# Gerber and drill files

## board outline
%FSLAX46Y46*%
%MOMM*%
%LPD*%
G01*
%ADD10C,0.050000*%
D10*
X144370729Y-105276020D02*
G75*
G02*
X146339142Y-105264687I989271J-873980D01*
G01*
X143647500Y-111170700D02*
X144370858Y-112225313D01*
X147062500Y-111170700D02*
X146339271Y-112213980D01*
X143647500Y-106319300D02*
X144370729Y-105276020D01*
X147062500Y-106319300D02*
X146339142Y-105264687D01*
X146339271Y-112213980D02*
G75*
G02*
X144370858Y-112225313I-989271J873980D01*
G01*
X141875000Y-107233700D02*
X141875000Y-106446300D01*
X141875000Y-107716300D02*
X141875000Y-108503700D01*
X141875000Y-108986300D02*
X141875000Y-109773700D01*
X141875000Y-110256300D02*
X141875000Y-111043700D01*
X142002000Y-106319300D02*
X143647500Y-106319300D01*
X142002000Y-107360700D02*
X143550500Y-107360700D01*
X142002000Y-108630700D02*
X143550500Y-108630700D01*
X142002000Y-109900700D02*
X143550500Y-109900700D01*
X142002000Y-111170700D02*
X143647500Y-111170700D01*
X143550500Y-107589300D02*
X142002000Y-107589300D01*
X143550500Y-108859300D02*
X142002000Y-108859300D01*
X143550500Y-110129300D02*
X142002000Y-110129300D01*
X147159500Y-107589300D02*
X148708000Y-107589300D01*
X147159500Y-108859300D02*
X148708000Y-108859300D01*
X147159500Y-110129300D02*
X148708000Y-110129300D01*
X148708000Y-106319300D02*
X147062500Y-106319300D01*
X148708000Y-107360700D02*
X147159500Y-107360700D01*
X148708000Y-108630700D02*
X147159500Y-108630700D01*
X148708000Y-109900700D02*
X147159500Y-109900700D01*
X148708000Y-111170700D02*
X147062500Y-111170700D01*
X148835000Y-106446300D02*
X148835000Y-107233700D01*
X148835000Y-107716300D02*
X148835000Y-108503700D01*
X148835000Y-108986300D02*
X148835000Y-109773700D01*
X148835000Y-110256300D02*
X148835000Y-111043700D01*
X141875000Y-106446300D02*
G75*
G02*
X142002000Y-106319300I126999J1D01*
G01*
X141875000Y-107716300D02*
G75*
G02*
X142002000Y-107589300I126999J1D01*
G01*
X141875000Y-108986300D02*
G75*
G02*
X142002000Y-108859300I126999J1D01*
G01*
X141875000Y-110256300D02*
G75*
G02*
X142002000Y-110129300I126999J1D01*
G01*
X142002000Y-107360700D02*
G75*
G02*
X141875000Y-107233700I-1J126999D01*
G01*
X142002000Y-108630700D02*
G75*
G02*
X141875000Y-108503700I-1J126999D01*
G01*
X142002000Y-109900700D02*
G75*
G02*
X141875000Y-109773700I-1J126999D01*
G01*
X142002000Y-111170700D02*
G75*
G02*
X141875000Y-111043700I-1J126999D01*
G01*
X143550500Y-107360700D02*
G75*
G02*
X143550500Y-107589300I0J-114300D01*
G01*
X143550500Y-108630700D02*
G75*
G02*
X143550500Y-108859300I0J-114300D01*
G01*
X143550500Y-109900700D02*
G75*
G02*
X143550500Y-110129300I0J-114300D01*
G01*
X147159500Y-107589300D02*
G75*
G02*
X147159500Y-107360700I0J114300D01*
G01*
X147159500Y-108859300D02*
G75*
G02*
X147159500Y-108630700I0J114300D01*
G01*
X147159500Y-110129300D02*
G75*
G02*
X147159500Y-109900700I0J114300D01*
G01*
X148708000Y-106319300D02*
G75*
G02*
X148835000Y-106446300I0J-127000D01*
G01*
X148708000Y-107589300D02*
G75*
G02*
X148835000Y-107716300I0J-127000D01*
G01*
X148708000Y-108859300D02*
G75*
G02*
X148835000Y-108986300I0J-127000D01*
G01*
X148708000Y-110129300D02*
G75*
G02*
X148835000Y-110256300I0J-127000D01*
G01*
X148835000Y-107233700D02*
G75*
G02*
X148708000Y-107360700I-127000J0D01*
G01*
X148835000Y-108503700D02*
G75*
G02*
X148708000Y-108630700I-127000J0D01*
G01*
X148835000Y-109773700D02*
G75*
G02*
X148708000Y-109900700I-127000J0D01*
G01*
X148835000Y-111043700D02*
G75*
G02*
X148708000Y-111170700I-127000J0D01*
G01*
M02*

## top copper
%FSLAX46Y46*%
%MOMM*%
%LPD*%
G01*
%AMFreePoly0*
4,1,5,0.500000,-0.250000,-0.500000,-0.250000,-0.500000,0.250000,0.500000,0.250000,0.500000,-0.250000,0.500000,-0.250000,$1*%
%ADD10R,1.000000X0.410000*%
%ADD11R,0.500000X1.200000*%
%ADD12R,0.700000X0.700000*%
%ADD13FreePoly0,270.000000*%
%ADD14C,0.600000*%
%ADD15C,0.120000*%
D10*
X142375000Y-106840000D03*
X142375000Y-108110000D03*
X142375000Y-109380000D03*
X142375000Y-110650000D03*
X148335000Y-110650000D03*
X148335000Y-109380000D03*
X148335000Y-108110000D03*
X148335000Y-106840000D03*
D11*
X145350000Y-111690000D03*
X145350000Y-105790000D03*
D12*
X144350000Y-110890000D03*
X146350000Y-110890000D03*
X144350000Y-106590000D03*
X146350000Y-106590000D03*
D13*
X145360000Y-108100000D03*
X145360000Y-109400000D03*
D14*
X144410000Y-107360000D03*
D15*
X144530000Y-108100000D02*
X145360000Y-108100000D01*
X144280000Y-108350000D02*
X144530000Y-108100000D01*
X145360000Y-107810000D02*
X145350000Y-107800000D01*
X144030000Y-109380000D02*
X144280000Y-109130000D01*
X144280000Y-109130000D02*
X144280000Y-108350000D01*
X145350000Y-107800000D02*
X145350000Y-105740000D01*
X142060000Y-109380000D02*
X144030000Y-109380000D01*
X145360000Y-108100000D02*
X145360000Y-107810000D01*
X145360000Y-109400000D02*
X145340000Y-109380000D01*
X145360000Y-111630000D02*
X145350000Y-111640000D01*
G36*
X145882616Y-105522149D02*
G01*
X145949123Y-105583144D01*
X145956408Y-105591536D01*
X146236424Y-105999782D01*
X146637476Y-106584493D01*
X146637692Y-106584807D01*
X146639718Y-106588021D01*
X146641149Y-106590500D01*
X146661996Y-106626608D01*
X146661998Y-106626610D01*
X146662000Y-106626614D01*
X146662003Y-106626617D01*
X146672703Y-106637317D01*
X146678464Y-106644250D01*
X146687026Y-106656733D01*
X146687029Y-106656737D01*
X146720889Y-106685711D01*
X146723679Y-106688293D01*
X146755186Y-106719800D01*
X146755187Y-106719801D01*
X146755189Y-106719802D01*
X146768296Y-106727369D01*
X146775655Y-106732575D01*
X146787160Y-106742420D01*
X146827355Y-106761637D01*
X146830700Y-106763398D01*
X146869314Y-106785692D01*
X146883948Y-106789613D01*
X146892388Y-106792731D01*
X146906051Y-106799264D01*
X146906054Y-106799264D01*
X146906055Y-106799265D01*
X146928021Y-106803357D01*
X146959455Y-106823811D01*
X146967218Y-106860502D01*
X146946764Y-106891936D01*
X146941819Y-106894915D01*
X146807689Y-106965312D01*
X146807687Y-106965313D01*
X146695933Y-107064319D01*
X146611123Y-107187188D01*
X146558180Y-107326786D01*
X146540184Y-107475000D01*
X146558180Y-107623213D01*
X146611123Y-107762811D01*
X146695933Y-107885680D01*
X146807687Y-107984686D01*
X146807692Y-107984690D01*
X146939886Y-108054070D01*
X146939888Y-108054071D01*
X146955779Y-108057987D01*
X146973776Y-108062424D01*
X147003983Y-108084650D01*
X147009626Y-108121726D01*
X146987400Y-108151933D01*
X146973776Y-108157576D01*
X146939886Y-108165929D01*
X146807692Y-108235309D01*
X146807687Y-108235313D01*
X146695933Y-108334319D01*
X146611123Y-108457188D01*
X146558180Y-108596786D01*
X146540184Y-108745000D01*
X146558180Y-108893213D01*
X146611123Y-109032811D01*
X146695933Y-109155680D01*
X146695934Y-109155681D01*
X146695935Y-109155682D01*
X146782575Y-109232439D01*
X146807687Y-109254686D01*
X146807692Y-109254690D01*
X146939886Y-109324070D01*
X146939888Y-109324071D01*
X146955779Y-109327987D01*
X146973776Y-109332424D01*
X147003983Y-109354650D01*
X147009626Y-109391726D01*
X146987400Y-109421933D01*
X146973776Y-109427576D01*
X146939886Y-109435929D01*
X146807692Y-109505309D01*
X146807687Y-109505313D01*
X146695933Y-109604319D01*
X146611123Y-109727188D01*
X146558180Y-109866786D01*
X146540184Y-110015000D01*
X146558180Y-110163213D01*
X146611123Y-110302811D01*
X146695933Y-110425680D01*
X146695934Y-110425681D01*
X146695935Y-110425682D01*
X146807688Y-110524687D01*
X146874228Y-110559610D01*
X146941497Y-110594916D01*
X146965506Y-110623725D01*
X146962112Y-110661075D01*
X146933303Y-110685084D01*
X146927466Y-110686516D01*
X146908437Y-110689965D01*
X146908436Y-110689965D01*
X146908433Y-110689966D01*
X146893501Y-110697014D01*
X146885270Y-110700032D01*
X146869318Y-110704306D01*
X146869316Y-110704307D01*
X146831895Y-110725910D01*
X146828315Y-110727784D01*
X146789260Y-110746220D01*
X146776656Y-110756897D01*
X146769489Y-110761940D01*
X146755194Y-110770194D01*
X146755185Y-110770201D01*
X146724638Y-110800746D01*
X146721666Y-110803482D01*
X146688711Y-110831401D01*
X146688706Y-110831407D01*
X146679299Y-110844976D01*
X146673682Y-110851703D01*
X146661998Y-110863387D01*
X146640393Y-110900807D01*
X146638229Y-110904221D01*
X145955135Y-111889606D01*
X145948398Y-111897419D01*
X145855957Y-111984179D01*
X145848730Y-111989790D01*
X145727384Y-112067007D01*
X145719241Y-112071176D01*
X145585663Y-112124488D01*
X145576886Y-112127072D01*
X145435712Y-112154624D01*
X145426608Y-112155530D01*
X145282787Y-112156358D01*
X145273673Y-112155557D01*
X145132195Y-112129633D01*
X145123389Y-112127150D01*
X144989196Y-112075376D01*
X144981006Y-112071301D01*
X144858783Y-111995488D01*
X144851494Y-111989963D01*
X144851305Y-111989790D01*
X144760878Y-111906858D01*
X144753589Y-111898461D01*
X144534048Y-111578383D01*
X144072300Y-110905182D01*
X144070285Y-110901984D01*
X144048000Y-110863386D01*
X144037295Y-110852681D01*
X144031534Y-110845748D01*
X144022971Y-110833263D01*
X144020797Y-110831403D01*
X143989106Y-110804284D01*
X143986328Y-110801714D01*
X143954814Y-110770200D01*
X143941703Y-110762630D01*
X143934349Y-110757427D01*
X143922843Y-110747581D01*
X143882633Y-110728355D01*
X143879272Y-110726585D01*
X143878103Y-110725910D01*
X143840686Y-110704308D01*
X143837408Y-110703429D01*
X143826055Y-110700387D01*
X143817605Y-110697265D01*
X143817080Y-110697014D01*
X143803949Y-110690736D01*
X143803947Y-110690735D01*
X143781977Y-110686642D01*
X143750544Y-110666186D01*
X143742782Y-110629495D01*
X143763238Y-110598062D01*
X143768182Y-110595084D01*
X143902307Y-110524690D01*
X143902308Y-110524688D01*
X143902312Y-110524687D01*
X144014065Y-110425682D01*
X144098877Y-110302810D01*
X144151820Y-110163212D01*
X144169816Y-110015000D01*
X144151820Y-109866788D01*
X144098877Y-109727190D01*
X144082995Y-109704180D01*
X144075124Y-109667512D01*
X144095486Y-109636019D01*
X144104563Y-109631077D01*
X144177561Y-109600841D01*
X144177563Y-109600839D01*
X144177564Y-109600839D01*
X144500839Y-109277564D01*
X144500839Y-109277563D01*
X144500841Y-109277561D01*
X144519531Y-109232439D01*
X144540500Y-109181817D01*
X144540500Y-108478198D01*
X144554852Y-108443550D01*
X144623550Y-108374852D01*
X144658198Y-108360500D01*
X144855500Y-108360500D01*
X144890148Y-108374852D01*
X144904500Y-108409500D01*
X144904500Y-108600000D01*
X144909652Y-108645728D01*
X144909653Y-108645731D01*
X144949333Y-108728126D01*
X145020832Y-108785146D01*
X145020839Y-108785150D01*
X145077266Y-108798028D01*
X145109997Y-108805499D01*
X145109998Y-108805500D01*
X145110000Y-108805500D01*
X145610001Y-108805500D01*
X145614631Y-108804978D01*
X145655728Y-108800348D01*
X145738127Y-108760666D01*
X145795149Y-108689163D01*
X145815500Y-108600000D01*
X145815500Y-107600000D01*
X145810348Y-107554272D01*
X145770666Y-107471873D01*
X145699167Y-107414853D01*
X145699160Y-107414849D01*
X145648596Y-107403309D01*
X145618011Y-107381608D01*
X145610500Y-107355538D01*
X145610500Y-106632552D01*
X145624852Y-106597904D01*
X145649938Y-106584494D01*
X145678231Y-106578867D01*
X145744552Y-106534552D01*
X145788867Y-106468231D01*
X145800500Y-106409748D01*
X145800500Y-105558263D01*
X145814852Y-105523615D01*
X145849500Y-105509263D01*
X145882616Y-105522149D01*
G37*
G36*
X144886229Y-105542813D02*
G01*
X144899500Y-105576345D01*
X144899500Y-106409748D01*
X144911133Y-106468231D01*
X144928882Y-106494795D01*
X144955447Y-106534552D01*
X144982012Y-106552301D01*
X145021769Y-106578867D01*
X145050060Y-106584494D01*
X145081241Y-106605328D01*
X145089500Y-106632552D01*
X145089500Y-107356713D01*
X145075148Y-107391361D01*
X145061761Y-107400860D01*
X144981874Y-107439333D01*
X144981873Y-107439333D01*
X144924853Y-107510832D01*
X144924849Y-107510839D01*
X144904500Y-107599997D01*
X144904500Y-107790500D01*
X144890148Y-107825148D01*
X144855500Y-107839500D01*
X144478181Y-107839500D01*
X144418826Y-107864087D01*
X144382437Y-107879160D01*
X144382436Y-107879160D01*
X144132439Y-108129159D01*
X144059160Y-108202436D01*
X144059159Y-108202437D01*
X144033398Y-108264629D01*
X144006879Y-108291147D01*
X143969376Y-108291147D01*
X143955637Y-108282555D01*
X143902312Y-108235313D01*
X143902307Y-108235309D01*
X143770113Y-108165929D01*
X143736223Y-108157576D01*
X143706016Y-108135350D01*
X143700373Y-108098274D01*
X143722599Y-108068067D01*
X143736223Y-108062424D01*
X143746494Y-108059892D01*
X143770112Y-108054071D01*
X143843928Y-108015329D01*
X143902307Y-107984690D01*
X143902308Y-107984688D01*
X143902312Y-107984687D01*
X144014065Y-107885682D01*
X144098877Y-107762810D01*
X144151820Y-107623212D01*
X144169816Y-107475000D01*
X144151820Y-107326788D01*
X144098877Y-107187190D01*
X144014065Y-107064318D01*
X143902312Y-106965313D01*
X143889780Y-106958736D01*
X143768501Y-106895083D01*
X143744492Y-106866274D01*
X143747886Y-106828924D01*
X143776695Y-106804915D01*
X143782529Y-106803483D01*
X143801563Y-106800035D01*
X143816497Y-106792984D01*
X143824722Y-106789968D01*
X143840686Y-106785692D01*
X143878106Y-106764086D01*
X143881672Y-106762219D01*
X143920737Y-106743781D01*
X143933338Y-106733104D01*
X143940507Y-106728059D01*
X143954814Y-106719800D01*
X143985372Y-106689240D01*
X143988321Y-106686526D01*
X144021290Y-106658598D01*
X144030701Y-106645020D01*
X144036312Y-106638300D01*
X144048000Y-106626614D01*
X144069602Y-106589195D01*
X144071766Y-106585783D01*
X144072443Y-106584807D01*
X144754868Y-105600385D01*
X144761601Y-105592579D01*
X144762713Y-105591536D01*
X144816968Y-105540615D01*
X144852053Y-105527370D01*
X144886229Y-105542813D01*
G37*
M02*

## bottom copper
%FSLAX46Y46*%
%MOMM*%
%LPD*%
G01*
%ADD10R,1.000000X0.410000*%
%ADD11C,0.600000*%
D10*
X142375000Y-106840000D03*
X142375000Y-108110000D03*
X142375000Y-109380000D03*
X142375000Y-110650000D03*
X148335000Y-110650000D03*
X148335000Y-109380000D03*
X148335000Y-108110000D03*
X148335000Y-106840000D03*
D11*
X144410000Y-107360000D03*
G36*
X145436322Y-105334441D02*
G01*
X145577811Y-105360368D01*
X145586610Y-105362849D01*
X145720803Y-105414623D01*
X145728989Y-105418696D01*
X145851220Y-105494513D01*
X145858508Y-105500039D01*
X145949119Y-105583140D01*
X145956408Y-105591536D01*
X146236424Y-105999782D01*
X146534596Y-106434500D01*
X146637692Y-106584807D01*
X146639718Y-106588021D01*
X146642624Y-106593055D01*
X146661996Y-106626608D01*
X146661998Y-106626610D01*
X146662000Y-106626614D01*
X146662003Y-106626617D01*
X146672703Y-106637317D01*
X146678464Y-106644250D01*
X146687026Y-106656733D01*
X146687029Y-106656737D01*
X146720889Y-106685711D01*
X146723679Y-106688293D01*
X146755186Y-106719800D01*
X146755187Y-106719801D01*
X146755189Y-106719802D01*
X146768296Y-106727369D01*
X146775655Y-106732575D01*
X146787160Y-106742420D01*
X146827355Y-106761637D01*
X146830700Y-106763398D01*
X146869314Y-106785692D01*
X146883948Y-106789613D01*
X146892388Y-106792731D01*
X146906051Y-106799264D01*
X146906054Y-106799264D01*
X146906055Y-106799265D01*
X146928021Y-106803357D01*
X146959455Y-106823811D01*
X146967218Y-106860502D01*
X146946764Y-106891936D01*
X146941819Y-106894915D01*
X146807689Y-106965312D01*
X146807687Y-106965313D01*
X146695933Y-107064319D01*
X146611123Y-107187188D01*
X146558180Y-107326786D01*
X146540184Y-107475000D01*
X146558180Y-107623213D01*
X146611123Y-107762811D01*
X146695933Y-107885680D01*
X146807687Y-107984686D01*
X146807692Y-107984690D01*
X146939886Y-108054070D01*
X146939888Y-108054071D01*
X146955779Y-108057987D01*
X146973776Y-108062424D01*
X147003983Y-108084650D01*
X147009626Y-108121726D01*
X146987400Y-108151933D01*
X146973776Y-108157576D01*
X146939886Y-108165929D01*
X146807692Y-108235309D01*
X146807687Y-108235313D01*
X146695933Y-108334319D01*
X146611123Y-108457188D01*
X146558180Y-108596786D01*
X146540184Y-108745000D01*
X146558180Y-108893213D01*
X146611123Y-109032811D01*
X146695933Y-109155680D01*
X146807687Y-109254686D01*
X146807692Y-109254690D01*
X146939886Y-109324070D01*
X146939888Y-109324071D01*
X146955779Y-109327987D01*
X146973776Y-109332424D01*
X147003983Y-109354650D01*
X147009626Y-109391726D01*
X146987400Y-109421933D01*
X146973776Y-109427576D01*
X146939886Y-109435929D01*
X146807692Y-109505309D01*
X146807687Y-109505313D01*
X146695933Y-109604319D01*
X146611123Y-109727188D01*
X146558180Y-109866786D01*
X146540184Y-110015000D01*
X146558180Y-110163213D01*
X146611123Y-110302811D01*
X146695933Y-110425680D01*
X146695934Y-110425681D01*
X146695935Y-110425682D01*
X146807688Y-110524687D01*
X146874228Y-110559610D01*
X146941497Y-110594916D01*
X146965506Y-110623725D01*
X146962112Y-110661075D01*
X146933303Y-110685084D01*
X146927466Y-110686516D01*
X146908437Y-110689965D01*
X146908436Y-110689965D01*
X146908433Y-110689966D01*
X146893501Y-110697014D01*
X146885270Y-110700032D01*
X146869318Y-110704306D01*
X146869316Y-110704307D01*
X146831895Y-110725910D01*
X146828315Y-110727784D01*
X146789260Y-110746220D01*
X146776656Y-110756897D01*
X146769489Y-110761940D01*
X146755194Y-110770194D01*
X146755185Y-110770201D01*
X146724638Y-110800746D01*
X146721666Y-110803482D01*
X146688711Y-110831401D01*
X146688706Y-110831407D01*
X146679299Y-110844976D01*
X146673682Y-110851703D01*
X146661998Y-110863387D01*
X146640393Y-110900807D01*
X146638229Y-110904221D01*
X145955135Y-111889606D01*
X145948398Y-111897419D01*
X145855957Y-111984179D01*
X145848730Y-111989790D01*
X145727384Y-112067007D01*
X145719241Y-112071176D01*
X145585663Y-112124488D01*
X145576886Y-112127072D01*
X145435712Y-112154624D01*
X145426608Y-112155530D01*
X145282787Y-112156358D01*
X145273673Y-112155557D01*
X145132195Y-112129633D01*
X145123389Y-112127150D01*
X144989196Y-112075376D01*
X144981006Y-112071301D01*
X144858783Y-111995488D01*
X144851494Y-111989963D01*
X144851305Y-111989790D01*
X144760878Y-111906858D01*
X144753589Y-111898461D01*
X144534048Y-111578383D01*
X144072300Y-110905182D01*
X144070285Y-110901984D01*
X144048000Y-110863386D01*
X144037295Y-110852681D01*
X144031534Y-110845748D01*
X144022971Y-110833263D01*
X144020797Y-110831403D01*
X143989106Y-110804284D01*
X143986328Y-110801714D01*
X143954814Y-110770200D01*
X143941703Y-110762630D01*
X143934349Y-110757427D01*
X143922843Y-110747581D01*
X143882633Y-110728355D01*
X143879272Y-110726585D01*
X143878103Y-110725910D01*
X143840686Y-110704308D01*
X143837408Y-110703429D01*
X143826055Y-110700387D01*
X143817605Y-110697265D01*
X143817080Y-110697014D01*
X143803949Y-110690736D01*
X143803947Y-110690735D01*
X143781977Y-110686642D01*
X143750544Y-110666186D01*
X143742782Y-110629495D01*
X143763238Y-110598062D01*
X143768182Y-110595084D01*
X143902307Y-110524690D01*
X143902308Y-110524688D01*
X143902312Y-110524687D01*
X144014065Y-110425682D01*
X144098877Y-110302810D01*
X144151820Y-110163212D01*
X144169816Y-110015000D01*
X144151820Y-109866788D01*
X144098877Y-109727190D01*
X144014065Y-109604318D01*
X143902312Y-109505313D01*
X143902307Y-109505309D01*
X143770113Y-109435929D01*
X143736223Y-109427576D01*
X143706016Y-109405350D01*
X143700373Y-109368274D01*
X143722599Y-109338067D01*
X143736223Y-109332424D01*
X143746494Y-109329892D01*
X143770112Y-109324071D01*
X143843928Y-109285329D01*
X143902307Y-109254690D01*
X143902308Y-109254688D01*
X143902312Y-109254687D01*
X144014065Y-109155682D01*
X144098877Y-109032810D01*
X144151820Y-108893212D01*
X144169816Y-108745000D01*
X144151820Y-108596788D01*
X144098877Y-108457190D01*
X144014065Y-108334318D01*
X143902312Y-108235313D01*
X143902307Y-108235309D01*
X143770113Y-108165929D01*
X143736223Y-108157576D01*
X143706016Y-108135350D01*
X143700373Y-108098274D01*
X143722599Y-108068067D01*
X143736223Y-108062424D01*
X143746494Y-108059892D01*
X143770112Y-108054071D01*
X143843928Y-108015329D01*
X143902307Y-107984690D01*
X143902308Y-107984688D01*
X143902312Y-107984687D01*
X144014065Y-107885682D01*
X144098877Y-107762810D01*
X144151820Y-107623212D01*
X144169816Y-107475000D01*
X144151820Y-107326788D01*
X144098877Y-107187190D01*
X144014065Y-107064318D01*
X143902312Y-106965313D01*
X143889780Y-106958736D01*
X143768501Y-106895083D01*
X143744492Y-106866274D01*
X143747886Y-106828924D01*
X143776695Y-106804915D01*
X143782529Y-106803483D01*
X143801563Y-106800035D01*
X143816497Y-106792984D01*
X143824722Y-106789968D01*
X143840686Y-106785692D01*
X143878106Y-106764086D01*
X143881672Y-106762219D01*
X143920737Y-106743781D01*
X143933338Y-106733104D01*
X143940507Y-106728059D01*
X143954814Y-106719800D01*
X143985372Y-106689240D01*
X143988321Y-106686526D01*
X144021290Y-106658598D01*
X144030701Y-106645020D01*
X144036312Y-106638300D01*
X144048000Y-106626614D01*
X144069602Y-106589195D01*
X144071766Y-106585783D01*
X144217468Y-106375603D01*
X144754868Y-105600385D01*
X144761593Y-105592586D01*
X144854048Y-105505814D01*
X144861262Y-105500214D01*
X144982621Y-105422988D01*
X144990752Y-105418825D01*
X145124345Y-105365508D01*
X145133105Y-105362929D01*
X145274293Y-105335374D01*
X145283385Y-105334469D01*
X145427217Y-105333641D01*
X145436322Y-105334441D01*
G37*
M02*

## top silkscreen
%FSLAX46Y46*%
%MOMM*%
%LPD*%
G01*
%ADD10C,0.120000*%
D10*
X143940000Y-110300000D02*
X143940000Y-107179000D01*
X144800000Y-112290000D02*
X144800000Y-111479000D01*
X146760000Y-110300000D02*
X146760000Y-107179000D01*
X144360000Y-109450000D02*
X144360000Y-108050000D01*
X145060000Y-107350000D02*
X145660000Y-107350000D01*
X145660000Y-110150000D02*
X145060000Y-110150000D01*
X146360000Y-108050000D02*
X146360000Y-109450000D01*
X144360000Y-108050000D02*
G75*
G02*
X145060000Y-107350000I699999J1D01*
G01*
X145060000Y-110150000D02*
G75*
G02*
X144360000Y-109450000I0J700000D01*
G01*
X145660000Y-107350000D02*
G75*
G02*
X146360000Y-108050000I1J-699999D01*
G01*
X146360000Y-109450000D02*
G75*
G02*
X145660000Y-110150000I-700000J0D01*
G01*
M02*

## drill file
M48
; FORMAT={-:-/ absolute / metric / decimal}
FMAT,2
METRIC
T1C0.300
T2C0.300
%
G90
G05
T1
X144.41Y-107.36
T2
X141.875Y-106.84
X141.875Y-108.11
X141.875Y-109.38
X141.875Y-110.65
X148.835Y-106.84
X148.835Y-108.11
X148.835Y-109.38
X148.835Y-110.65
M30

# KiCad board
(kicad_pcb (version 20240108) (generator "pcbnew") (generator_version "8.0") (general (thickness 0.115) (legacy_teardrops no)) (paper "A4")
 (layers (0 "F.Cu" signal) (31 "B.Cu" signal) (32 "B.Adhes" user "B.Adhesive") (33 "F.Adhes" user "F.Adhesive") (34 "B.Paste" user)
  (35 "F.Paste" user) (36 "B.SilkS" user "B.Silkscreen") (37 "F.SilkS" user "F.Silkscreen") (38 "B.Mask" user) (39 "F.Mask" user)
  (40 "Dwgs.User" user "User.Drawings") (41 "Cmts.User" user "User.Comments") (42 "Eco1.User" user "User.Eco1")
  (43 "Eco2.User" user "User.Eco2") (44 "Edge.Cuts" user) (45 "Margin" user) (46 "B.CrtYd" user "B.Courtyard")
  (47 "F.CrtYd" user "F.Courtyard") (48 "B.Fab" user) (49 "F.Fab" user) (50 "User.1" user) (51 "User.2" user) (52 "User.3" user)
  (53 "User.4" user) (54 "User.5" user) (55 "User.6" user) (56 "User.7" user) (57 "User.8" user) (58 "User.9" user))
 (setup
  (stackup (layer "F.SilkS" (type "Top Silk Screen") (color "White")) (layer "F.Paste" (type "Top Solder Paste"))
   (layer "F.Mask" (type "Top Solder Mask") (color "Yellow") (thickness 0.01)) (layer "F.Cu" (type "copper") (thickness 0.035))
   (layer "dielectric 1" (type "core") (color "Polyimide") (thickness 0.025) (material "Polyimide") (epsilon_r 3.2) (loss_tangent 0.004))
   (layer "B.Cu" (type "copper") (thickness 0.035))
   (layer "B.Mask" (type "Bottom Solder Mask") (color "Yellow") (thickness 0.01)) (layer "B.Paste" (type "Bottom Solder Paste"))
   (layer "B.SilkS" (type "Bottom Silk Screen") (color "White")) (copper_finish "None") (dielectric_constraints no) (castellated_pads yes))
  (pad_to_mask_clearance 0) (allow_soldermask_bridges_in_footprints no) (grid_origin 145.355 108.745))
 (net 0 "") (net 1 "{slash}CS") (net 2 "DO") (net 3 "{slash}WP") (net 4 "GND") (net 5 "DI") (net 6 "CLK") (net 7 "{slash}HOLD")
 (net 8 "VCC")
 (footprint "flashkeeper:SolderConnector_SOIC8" (layer "F.Cu") (at 145.355 108.745)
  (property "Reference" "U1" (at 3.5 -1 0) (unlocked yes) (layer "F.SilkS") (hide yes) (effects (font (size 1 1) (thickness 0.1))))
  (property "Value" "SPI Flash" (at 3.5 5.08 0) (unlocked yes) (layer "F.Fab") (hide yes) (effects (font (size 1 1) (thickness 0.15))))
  (fp_line (start -3.48 -1.5113) (end -3.48 -2.2987) (stroke (width 0.05) (type default)) (layer "Edge.Cuts"))
  (fp_line (start -3.48 -1.0287) (end -3.48 -0.2413) (stroke (width 0.05) (type default)) (layer "Edge.Cuts"))
  (fp_line (start -3.48 0.2413) (end -3.48 1.0287) (stroke (width 0.05) (type default)) (layer "Edge.Cuts"))
  (fp_line (start -3.48 1.5113) (end -3.48 2.2987) (stroke (width 0.05) (type default)) (layer "Edge.Cuts"))
  (fp_line (start -3.353 -2.4257) (end -1.7075 -2.4257) (stroke (width 0.05) (type default)) (layer "Edge.Cuts"))
  (fp_line (start -3.353 -1.3843) (end -1.8045 -1.3843) (stroke (width 0.05) (type default)) (layer "Edge.Cuts"))
  (fp_line (start -3.353 -0.1143) (end -1.8045 -0.1143) (stroke (width 0.05) (type default)) (layer "Edge.Cuts"))
  (fp_line (start -3.353 1.1557) (end -1.8045 1.1557) (stroke (width 0.05) (type default)) (layer "Edge.Cuts"))
  (fp_line (start -3.353 2.4257) (end -1.7075 2.4257) (stroke (width 0.05) (type default)) (layer "Edge.Cuts"))
  (fp_line (start -1.8045 -1.1557) (end -3.353 -1.1557) (stroke (width 0.05) (type default)) (layer "Edge.Cuts"))
  (fp_line (start -1.8045 0.1143) (end -3.353 0.1143) (stroke (width 0.05) (type default)) (layer "Edge.Cuts"))
  (fp_line (start -1.8045 1.3843) (end -3.353 1.3843) (stroke (width 0.05) (type default)) (layer "Edge.Cuts"))
  (fp_line (start 1.8045 -1.1557) (end 3.353 -1.1557) (stroke (width 0.05) (type default)) (layer "Edge.Cuts"))
  (fp_line (start 1.8045 0.1143) (end 3.353 0.1143) (stroke (width 0.05) (type default)) (layer "Edge.Cuts"))
  (fp_line (start 1.8045 1.3843) (end 3.353 1.3843) (stroke (width 0.05) (type default)) (layer "Edge.Cuts"))
  (fp_line (start 3.353 -2.4257) (end 1.7075 -2.4257) (stroke (width 0.05) (type default)) (layer "Edge.Cuts"))
  (fp_line (start 3.353 -1.3843) (end 1.8045 -1.3843) (stroke (width 0.05) (type default)) (layer "Edge.Cuts"))
  (fp_line (start 3.353 -0.1143) (end 1.8045 -0.1143) (stroke (width 0.05) (type default)) (layer "Edge.Cuts"))
  (fp_line (start 3.353 1.1557) (end 1.8045 1.1557) (stroke (width 0.05) (type default)) (layer "Edge.Cuts"))
  (fp_line (start 3.353 2.4257) (end 1.7075 2.4257) (stroke (width 0.05) (type default)) (layer "Edge.Cuts"))
  (fp_line (start 3.48 -2.2987) (end 3.48 -1.5113) (stroke (width 0.05) (type default)) (layer "Edge.Cuts"))
  (fp_line (start 3.48 -1.0287) (end 3.48 -0.2413) (stroke (width 0.05) (type default)) (layer "Edge.Cuts"))
  (fp_line (start 3.48 0.2413) (end 3.48 1.0287) (stroke (width 0.05) (type default)) (layer "Edge.Cuts"))
  (fp_line (start 3.48 1.5113) (end 3.48 2.2987) (stroke (width 0.05) (type default)) (layer "Edge.Cuts"))
  (fp_arc (start -3.48 -2.2987) (mid -3.442803 -2.388503) (end -3.353 -2.4257) (stroke (width 0.05) (type default)) (layer "Edge.Cuts"))
  (fp_arc (start -3.48 -1.0287) (mid -3.442803 -1.118503) (end -3.353 -1.1557) (stroke (width 0.05) (type default)) (layer "Edge.Cuts"))
  (fp_arc (start -3.48 0.2413) (mid -3.442803 0.151497) (end -3.353 0.1143) (stroke (width 0.05) (type default)) (layer "Edge.Cuts"))
  (fp_arc (start -3.48 1.5113) (mid -3.442803 1.421497) (end -3.353 1.3843) (stroke (width 0.05) (type default)) (layer "Edge.Cuts"))
  (fp_arc (start -3.353 -1.3843) (mid -3.442803 -1.421497) (end -3.48 -1.5113) (stroke (width 0.05) (type default)) (layer "Edge.Cuts"))
  (fp_arc (start -3.353 -0.1143) (mid -3.442803 -0.151497) (end -3.48 -0.2413) (stroke (width 0.05) (type default)) (layer "Edge.Cuts"))
  (fp_arc (start -3.353 1.1557) (mid -3.442803 1.118503) (end -3.48 1.0287) (stroke (width 0.05) (type default)) (layer "Edge.Cuts"))
  (fp_arc (start -3.353 2.4257) (mid -3.442803 2.388503) (end -3.48 2.2987) (stroke (width 0.05) (type default)) (layer "Edge.Cuts"))
  (fp_arc (start -1.8045 -1.3843) (mid -1.6902 -1.27) (end -1.8045 -1.1557) (stroke (width 0.05) (type default)) (layer "Edge.Cuts"))
  (fp_arc (start -1.8045 -0.1143) (mid -1.6902 0) (end -1.8045 0.1143) (stroke (width 0.05) (type default)) (layer "Edge.Cuts"))
  (fp_arc (start -1.8045 1.1557) (mid -1.6902 1.27) (end -1.8045 1.3843) (stroke (width 0.05) (type default)) (layer "Edge.Cuts"))
  (fp_arc (start 1.8045 -1.1557) (mid 1.6902 -1.27) (end 1.8045 -1.3843) (stroke (width 0.05) (type default)) (layer "Edge.Cuts"))
  (fp_arc (start 1.8045 0.1143) (mid 1.6902 0) (end 1.8045 -0.1143) (stroke (width 0.05) (type default)) (layer "Edge.Cuts"))
  (fp_arc (start 1.8045 1.3843) (mid 1.6902 1.27) (end 1.8045 1.1557) (stroke (width 0.05) (type default)) (layer "Edge.Cuts"))
  (fp_arc (start 3.353 -2.4257) (mid 3.442803 -2.388503) (end 3.48 -2.2987) (stroke (width 0.05) (type default)) (layer "Edge.Cuts"))
  (fp_arc (start 3.353 -1.1557) (mid 3.442803 -1.118503) (end 3.48 -1.0287) (stroke (width 0.05) (type default)) (layer "Edge.Cuts"))
  (fp_arc (start 3.353 0.1143) (mid 3.442803 0.151497) (end 3.48 0.2413) (stroke (width 0.05) (type default)) (layer "Edge.Cuts"))
  (fp_arc (start 3.353 1.3843) (mid 3.442803 1.421497) (end 3.48 1.5113) (stroke (width 0.05) (type default)) (layer "Edge.Cuts"))
  (fp_arc (start 3.48 -1.5113) (mid 3.442803 -1.421497) (end 3.353 -1.3843) (stroke (width 0.05) (type default)) (layer "Edge.Cuts"))
  (fp_arc (start 3.48 -0.2413) (mid 3.442803 -0.151497) (end 3.353 -0.1143) (stroke (width 0.05) (type default)) (layer "Edge.Cuts"))
  (fp_arc (start 3.48 1.0287) (mid 3.442803 1.118503) (end 3.353 1.1557) (stroke (width 0.05) (type default)) (layer "Edge.Cuts"))
  (fp_arc (start 3.48 2.2987) (mid 3.442803 2.388503) (end 3.353 2.4257) (stroke (width 0.05) (type default)) (layer "Edge.Cuts"))
  (pad "1" thru_hole rect (at -3.48 -1.905) (size 1 0.41) (drill 0.3 (offset 0.5 0)) (layers "*.Cu" "*.Mask") (remove_unused_layers no)
   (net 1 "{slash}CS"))
  (pad "2" thru_hole rect (at -3.48 -0.635) (size 1 0.41) (drill 0.3 (offset 0.5 0)) (layers "*.Cu" "*.Mask") (remove_unused_layers no)
   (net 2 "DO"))
  (pad "3" thru_hole rect (at -3.48 0.635) (size 1 0.41) (drill 0.3 (offset 0.5 0)) (layers "*.Cu" "*.Mask") (remove_unused_layers no)
   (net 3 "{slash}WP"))
  (pad "4" thru_hole rect (at -3.48 1.905) (size 1 0.41) (drill 0.3 (offset 0.5 0)) (layers "*.Cu" "*.Mask") (remove_unused_layers no)
   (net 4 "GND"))
  (pad "5" thru_hole rect (at 3.48 1.905 180) (size 1 0.41) (drill 0.3 (offset 0.5 0)) (layers "*.Cu" "*.Mask") (remove_unused_layers no)
   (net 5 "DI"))
  (pad "6" thru_hole rect (at 3.48 0.635 180) (size 1 0.41) (drill 0.3 (offset 0.5 0)) (layers "*.Cu" "*.Mask") (remove_unused_layers no)
   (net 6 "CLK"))
  (pad "7" thru_hole rect (at 3.48 -0.635 180) (size 1 0.41) (drill 0.3 (offset 0.5 0)) (layers "*.Cu" "*.Mask") (remove_unused_layers no)
   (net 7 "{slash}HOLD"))
  (pad "8" thru_hole rect (at 3.48 -1.905 180) (size 1 0.41) (drill 0.3 (offset 0.5 0)) (layers "*.Cu" "*.Mask") (remove_unused_layers no)
   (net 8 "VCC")))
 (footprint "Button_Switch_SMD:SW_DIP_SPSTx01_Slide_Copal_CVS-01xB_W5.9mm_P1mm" (layer "F.Cu") (at 145.35 108.74 90)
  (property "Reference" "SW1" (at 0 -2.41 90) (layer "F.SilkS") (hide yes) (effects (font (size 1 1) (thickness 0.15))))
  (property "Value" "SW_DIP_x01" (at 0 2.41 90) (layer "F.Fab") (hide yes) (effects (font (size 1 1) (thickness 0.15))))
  (fp_line (start -1.56 -1.41) (end 1.561 -1.41) (stroke (width 0.12) (type solid)) (layer "F.SilkS"))
  (fp_line (start -3.55 -0.55) (end -2.739 -0.55) (stroke (width 0.12) (type solid)) (layer "F.SilkS"))
  (fp_line (start -1.56 1.41) (end 1.561 1.41) (stroke (width 0.12) (type solid)) (layer "F.SilkS"))
  (pad "1" smd rect (at -2.95 0 90) (size 1.2 0.5) (layers "F.Cu" "F.Paste" "F.Mask") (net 4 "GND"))
  (pad "2" smd rect (at 2.95 0 90) (size 1.2 0.5) (layers "F.Cu" "F.Paste" "F.Mask") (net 3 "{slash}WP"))
  (pad "3" smd rect (at -2.15 -1 90) (size 0.7 0.7) (layers "F.Cu" "F.Paste" "F.Mask") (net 4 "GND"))
  (pad "3" smd rect (at -2.15 1 90) (size 0.7 0.7) (layers "F.Cu" "F.Paste" "F.Mask") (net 4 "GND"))
  (pad "3" smd rect (at 2.15 -1 90) (size 0.7 0.7) (layers "F.Cu" "F.Paste" "F.Mask") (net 4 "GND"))
  (pad "3" smd rect (at 2.15 1 90) (size 0.7 0.7) (layers "F.Cu" "F.Paste" "F.Mask") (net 4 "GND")))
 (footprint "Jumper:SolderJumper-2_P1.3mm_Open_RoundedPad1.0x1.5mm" (layer "F.Cu") (at 145.36 108.75 -90)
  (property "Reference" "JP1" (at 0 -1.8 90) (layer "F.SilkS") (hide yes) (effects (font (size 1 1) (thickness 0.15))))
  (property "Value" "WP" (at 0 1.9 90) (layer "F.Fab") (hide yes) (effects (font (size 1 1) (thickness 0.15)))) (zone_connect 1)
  (fp_line (start 0.7 1) (end -0.7 1) (stroke (width 0.12) (type solid)) (layer "F.SilkS"))
  (fp_line (start -1.4 0.3) (end -1.4 -0.3) (stroke (width 0.12) (type solid)) (layer "F.SilkS"))
  (fp_line (start 1.4 -0.3) (end 1.4 0.3) (stroke (width 0.12) (type solid)) (layer "F.SilkS"))
  (fp_line (start -0.7 -1) (end 0.7 -1) (stroke (width 0.12) (type solid)) (layer "F.SilkS"))
  (fp_arc (start -0.7 1) (mid -1.194975 0.794975) (end -1.4 0.3) (stroke (width 0.12) (type solid)) (layer "F.SilkS"))
  (fp_arc (start 1.4 0.3) (mid 1.194975 0.794975) (end 0.7 1) (stroke (width 0.12) (type solid)) (layer "F.SilkS"))
  (fp_arc (start -1.4 -0.3) (mid -1.194975 -0.794975) (end -0.7 -1) (stroke (width 0.12) (type solid)) (layer "F.SilkS"))
  (fp_arc (start 0.7 -1) (mid 1.194975 -0.794975) (end 1.4 -0.3) (stroke (width 0.12) (type solid)) (layer "F.SilkS"))
  (pad "1" smd custom (at -0.65 0 270) (size 1 0.5) (layers "F.Cu" "F.Mask") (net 3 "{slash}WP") (zone_connect 2) (thermal_bridge_angle 45)
   (options (clearance outline) (anchor rect)) (primitives))
  (pad "2" smd custom (at 0.65 0 270) (size 1 0.5) (layers "F.Cu" "F.Mask") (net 4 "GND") (zone_connect 2) (thermal_bridge_angle 45)
   (options (clearance outline) (anchor rect)) (primitives)))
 (gr_arc (start 144.370729 105.27602) (mid 145.3524 104.829985) (end 146.339142 105.264687) (stroke (width 0.05) (type default))
  (layer "Edge.Cuts"))
 (gr_line (start 143.6475 111.1707) (end 144.370858 112.225313) (stroke (width 0.05) (type default)) (layer "Edge.Cuts"))
 (gr_line (start 147.0625 111.1707) (end 146.339271 112.21398) (stroke (width 0.05) (type default)) (layer "Edge.Cuts"))
 (gr_line (start 143.6475 106.3193) (end 144.370729 105.27602) (stroke (width 0.05) (type default)) (layer "Edge.Cuts"))
 (gr_line (start 147.0625 106.3193) (end 146.339142 105.264687) (stroke (width 0.05) (type default)) (layer "Edge.Cuts"))
 (gr_arc (start 146.339271 112.21398) (mid 145.3576 112.660015) (end 144.370858 112.225313) (stroke (width 0.05) (type default))
  (layer "Edge.Cuts"))
 (segment (start 144.53 108.1) (end 145.36 108.1) (width 0.12) (layer "F.Cu") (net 3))
 (segment (start 144.28 108.35) (end 144.53 108.1) (width 0.12) (layer "F.Cu") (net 3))
 (segment (start 145.36 107.81) (end 145.35 107.8) (width 0.12) (layer "F.Cu") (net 3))
 (segment (start 144.03 109.38) (end 144.28 109.13) (width 0.12) (layer "F.Cu") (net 3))
 (segment (start 144.28 109.13) (end 144.28 108.35) (width 0.12) (layer "F.Cu") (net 3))
 (segment (start 145.35 107.8) (end 145.35 105.74) (width 0.12) (layer "F.Cu") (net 3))
 (segment (start 142.06 109.38) (end 144.03 109.38) (width 0.12) (layer "F.Cu") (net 3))
 (segment (start 145.36 108.1) (end 145.36 107.81) (width 0.12) (layer "F.Cu") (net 3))
 (segment (start 145.36 109.4) (end 145.34 109.38) (width 0.12) (layer "F.Cu") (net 4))
 (segment (start 145.36 111.63) (end 145.35 111.64) (width 0.12) (layer "F.Cu") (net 4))
 (via (at 144.41 107.36) (size 0.6) (drill 0.3) (layers "F.Cu" "B.Cu") (free yes) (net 4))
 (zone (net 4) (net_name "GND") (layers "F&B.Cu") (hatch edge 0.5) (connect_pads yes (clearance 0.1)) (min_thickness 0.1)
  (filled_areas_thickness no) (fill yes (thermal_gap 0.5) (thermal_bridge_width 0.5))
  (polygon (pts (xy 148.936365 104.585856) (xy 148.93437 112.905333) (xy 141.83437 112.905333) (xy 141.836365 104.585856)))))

